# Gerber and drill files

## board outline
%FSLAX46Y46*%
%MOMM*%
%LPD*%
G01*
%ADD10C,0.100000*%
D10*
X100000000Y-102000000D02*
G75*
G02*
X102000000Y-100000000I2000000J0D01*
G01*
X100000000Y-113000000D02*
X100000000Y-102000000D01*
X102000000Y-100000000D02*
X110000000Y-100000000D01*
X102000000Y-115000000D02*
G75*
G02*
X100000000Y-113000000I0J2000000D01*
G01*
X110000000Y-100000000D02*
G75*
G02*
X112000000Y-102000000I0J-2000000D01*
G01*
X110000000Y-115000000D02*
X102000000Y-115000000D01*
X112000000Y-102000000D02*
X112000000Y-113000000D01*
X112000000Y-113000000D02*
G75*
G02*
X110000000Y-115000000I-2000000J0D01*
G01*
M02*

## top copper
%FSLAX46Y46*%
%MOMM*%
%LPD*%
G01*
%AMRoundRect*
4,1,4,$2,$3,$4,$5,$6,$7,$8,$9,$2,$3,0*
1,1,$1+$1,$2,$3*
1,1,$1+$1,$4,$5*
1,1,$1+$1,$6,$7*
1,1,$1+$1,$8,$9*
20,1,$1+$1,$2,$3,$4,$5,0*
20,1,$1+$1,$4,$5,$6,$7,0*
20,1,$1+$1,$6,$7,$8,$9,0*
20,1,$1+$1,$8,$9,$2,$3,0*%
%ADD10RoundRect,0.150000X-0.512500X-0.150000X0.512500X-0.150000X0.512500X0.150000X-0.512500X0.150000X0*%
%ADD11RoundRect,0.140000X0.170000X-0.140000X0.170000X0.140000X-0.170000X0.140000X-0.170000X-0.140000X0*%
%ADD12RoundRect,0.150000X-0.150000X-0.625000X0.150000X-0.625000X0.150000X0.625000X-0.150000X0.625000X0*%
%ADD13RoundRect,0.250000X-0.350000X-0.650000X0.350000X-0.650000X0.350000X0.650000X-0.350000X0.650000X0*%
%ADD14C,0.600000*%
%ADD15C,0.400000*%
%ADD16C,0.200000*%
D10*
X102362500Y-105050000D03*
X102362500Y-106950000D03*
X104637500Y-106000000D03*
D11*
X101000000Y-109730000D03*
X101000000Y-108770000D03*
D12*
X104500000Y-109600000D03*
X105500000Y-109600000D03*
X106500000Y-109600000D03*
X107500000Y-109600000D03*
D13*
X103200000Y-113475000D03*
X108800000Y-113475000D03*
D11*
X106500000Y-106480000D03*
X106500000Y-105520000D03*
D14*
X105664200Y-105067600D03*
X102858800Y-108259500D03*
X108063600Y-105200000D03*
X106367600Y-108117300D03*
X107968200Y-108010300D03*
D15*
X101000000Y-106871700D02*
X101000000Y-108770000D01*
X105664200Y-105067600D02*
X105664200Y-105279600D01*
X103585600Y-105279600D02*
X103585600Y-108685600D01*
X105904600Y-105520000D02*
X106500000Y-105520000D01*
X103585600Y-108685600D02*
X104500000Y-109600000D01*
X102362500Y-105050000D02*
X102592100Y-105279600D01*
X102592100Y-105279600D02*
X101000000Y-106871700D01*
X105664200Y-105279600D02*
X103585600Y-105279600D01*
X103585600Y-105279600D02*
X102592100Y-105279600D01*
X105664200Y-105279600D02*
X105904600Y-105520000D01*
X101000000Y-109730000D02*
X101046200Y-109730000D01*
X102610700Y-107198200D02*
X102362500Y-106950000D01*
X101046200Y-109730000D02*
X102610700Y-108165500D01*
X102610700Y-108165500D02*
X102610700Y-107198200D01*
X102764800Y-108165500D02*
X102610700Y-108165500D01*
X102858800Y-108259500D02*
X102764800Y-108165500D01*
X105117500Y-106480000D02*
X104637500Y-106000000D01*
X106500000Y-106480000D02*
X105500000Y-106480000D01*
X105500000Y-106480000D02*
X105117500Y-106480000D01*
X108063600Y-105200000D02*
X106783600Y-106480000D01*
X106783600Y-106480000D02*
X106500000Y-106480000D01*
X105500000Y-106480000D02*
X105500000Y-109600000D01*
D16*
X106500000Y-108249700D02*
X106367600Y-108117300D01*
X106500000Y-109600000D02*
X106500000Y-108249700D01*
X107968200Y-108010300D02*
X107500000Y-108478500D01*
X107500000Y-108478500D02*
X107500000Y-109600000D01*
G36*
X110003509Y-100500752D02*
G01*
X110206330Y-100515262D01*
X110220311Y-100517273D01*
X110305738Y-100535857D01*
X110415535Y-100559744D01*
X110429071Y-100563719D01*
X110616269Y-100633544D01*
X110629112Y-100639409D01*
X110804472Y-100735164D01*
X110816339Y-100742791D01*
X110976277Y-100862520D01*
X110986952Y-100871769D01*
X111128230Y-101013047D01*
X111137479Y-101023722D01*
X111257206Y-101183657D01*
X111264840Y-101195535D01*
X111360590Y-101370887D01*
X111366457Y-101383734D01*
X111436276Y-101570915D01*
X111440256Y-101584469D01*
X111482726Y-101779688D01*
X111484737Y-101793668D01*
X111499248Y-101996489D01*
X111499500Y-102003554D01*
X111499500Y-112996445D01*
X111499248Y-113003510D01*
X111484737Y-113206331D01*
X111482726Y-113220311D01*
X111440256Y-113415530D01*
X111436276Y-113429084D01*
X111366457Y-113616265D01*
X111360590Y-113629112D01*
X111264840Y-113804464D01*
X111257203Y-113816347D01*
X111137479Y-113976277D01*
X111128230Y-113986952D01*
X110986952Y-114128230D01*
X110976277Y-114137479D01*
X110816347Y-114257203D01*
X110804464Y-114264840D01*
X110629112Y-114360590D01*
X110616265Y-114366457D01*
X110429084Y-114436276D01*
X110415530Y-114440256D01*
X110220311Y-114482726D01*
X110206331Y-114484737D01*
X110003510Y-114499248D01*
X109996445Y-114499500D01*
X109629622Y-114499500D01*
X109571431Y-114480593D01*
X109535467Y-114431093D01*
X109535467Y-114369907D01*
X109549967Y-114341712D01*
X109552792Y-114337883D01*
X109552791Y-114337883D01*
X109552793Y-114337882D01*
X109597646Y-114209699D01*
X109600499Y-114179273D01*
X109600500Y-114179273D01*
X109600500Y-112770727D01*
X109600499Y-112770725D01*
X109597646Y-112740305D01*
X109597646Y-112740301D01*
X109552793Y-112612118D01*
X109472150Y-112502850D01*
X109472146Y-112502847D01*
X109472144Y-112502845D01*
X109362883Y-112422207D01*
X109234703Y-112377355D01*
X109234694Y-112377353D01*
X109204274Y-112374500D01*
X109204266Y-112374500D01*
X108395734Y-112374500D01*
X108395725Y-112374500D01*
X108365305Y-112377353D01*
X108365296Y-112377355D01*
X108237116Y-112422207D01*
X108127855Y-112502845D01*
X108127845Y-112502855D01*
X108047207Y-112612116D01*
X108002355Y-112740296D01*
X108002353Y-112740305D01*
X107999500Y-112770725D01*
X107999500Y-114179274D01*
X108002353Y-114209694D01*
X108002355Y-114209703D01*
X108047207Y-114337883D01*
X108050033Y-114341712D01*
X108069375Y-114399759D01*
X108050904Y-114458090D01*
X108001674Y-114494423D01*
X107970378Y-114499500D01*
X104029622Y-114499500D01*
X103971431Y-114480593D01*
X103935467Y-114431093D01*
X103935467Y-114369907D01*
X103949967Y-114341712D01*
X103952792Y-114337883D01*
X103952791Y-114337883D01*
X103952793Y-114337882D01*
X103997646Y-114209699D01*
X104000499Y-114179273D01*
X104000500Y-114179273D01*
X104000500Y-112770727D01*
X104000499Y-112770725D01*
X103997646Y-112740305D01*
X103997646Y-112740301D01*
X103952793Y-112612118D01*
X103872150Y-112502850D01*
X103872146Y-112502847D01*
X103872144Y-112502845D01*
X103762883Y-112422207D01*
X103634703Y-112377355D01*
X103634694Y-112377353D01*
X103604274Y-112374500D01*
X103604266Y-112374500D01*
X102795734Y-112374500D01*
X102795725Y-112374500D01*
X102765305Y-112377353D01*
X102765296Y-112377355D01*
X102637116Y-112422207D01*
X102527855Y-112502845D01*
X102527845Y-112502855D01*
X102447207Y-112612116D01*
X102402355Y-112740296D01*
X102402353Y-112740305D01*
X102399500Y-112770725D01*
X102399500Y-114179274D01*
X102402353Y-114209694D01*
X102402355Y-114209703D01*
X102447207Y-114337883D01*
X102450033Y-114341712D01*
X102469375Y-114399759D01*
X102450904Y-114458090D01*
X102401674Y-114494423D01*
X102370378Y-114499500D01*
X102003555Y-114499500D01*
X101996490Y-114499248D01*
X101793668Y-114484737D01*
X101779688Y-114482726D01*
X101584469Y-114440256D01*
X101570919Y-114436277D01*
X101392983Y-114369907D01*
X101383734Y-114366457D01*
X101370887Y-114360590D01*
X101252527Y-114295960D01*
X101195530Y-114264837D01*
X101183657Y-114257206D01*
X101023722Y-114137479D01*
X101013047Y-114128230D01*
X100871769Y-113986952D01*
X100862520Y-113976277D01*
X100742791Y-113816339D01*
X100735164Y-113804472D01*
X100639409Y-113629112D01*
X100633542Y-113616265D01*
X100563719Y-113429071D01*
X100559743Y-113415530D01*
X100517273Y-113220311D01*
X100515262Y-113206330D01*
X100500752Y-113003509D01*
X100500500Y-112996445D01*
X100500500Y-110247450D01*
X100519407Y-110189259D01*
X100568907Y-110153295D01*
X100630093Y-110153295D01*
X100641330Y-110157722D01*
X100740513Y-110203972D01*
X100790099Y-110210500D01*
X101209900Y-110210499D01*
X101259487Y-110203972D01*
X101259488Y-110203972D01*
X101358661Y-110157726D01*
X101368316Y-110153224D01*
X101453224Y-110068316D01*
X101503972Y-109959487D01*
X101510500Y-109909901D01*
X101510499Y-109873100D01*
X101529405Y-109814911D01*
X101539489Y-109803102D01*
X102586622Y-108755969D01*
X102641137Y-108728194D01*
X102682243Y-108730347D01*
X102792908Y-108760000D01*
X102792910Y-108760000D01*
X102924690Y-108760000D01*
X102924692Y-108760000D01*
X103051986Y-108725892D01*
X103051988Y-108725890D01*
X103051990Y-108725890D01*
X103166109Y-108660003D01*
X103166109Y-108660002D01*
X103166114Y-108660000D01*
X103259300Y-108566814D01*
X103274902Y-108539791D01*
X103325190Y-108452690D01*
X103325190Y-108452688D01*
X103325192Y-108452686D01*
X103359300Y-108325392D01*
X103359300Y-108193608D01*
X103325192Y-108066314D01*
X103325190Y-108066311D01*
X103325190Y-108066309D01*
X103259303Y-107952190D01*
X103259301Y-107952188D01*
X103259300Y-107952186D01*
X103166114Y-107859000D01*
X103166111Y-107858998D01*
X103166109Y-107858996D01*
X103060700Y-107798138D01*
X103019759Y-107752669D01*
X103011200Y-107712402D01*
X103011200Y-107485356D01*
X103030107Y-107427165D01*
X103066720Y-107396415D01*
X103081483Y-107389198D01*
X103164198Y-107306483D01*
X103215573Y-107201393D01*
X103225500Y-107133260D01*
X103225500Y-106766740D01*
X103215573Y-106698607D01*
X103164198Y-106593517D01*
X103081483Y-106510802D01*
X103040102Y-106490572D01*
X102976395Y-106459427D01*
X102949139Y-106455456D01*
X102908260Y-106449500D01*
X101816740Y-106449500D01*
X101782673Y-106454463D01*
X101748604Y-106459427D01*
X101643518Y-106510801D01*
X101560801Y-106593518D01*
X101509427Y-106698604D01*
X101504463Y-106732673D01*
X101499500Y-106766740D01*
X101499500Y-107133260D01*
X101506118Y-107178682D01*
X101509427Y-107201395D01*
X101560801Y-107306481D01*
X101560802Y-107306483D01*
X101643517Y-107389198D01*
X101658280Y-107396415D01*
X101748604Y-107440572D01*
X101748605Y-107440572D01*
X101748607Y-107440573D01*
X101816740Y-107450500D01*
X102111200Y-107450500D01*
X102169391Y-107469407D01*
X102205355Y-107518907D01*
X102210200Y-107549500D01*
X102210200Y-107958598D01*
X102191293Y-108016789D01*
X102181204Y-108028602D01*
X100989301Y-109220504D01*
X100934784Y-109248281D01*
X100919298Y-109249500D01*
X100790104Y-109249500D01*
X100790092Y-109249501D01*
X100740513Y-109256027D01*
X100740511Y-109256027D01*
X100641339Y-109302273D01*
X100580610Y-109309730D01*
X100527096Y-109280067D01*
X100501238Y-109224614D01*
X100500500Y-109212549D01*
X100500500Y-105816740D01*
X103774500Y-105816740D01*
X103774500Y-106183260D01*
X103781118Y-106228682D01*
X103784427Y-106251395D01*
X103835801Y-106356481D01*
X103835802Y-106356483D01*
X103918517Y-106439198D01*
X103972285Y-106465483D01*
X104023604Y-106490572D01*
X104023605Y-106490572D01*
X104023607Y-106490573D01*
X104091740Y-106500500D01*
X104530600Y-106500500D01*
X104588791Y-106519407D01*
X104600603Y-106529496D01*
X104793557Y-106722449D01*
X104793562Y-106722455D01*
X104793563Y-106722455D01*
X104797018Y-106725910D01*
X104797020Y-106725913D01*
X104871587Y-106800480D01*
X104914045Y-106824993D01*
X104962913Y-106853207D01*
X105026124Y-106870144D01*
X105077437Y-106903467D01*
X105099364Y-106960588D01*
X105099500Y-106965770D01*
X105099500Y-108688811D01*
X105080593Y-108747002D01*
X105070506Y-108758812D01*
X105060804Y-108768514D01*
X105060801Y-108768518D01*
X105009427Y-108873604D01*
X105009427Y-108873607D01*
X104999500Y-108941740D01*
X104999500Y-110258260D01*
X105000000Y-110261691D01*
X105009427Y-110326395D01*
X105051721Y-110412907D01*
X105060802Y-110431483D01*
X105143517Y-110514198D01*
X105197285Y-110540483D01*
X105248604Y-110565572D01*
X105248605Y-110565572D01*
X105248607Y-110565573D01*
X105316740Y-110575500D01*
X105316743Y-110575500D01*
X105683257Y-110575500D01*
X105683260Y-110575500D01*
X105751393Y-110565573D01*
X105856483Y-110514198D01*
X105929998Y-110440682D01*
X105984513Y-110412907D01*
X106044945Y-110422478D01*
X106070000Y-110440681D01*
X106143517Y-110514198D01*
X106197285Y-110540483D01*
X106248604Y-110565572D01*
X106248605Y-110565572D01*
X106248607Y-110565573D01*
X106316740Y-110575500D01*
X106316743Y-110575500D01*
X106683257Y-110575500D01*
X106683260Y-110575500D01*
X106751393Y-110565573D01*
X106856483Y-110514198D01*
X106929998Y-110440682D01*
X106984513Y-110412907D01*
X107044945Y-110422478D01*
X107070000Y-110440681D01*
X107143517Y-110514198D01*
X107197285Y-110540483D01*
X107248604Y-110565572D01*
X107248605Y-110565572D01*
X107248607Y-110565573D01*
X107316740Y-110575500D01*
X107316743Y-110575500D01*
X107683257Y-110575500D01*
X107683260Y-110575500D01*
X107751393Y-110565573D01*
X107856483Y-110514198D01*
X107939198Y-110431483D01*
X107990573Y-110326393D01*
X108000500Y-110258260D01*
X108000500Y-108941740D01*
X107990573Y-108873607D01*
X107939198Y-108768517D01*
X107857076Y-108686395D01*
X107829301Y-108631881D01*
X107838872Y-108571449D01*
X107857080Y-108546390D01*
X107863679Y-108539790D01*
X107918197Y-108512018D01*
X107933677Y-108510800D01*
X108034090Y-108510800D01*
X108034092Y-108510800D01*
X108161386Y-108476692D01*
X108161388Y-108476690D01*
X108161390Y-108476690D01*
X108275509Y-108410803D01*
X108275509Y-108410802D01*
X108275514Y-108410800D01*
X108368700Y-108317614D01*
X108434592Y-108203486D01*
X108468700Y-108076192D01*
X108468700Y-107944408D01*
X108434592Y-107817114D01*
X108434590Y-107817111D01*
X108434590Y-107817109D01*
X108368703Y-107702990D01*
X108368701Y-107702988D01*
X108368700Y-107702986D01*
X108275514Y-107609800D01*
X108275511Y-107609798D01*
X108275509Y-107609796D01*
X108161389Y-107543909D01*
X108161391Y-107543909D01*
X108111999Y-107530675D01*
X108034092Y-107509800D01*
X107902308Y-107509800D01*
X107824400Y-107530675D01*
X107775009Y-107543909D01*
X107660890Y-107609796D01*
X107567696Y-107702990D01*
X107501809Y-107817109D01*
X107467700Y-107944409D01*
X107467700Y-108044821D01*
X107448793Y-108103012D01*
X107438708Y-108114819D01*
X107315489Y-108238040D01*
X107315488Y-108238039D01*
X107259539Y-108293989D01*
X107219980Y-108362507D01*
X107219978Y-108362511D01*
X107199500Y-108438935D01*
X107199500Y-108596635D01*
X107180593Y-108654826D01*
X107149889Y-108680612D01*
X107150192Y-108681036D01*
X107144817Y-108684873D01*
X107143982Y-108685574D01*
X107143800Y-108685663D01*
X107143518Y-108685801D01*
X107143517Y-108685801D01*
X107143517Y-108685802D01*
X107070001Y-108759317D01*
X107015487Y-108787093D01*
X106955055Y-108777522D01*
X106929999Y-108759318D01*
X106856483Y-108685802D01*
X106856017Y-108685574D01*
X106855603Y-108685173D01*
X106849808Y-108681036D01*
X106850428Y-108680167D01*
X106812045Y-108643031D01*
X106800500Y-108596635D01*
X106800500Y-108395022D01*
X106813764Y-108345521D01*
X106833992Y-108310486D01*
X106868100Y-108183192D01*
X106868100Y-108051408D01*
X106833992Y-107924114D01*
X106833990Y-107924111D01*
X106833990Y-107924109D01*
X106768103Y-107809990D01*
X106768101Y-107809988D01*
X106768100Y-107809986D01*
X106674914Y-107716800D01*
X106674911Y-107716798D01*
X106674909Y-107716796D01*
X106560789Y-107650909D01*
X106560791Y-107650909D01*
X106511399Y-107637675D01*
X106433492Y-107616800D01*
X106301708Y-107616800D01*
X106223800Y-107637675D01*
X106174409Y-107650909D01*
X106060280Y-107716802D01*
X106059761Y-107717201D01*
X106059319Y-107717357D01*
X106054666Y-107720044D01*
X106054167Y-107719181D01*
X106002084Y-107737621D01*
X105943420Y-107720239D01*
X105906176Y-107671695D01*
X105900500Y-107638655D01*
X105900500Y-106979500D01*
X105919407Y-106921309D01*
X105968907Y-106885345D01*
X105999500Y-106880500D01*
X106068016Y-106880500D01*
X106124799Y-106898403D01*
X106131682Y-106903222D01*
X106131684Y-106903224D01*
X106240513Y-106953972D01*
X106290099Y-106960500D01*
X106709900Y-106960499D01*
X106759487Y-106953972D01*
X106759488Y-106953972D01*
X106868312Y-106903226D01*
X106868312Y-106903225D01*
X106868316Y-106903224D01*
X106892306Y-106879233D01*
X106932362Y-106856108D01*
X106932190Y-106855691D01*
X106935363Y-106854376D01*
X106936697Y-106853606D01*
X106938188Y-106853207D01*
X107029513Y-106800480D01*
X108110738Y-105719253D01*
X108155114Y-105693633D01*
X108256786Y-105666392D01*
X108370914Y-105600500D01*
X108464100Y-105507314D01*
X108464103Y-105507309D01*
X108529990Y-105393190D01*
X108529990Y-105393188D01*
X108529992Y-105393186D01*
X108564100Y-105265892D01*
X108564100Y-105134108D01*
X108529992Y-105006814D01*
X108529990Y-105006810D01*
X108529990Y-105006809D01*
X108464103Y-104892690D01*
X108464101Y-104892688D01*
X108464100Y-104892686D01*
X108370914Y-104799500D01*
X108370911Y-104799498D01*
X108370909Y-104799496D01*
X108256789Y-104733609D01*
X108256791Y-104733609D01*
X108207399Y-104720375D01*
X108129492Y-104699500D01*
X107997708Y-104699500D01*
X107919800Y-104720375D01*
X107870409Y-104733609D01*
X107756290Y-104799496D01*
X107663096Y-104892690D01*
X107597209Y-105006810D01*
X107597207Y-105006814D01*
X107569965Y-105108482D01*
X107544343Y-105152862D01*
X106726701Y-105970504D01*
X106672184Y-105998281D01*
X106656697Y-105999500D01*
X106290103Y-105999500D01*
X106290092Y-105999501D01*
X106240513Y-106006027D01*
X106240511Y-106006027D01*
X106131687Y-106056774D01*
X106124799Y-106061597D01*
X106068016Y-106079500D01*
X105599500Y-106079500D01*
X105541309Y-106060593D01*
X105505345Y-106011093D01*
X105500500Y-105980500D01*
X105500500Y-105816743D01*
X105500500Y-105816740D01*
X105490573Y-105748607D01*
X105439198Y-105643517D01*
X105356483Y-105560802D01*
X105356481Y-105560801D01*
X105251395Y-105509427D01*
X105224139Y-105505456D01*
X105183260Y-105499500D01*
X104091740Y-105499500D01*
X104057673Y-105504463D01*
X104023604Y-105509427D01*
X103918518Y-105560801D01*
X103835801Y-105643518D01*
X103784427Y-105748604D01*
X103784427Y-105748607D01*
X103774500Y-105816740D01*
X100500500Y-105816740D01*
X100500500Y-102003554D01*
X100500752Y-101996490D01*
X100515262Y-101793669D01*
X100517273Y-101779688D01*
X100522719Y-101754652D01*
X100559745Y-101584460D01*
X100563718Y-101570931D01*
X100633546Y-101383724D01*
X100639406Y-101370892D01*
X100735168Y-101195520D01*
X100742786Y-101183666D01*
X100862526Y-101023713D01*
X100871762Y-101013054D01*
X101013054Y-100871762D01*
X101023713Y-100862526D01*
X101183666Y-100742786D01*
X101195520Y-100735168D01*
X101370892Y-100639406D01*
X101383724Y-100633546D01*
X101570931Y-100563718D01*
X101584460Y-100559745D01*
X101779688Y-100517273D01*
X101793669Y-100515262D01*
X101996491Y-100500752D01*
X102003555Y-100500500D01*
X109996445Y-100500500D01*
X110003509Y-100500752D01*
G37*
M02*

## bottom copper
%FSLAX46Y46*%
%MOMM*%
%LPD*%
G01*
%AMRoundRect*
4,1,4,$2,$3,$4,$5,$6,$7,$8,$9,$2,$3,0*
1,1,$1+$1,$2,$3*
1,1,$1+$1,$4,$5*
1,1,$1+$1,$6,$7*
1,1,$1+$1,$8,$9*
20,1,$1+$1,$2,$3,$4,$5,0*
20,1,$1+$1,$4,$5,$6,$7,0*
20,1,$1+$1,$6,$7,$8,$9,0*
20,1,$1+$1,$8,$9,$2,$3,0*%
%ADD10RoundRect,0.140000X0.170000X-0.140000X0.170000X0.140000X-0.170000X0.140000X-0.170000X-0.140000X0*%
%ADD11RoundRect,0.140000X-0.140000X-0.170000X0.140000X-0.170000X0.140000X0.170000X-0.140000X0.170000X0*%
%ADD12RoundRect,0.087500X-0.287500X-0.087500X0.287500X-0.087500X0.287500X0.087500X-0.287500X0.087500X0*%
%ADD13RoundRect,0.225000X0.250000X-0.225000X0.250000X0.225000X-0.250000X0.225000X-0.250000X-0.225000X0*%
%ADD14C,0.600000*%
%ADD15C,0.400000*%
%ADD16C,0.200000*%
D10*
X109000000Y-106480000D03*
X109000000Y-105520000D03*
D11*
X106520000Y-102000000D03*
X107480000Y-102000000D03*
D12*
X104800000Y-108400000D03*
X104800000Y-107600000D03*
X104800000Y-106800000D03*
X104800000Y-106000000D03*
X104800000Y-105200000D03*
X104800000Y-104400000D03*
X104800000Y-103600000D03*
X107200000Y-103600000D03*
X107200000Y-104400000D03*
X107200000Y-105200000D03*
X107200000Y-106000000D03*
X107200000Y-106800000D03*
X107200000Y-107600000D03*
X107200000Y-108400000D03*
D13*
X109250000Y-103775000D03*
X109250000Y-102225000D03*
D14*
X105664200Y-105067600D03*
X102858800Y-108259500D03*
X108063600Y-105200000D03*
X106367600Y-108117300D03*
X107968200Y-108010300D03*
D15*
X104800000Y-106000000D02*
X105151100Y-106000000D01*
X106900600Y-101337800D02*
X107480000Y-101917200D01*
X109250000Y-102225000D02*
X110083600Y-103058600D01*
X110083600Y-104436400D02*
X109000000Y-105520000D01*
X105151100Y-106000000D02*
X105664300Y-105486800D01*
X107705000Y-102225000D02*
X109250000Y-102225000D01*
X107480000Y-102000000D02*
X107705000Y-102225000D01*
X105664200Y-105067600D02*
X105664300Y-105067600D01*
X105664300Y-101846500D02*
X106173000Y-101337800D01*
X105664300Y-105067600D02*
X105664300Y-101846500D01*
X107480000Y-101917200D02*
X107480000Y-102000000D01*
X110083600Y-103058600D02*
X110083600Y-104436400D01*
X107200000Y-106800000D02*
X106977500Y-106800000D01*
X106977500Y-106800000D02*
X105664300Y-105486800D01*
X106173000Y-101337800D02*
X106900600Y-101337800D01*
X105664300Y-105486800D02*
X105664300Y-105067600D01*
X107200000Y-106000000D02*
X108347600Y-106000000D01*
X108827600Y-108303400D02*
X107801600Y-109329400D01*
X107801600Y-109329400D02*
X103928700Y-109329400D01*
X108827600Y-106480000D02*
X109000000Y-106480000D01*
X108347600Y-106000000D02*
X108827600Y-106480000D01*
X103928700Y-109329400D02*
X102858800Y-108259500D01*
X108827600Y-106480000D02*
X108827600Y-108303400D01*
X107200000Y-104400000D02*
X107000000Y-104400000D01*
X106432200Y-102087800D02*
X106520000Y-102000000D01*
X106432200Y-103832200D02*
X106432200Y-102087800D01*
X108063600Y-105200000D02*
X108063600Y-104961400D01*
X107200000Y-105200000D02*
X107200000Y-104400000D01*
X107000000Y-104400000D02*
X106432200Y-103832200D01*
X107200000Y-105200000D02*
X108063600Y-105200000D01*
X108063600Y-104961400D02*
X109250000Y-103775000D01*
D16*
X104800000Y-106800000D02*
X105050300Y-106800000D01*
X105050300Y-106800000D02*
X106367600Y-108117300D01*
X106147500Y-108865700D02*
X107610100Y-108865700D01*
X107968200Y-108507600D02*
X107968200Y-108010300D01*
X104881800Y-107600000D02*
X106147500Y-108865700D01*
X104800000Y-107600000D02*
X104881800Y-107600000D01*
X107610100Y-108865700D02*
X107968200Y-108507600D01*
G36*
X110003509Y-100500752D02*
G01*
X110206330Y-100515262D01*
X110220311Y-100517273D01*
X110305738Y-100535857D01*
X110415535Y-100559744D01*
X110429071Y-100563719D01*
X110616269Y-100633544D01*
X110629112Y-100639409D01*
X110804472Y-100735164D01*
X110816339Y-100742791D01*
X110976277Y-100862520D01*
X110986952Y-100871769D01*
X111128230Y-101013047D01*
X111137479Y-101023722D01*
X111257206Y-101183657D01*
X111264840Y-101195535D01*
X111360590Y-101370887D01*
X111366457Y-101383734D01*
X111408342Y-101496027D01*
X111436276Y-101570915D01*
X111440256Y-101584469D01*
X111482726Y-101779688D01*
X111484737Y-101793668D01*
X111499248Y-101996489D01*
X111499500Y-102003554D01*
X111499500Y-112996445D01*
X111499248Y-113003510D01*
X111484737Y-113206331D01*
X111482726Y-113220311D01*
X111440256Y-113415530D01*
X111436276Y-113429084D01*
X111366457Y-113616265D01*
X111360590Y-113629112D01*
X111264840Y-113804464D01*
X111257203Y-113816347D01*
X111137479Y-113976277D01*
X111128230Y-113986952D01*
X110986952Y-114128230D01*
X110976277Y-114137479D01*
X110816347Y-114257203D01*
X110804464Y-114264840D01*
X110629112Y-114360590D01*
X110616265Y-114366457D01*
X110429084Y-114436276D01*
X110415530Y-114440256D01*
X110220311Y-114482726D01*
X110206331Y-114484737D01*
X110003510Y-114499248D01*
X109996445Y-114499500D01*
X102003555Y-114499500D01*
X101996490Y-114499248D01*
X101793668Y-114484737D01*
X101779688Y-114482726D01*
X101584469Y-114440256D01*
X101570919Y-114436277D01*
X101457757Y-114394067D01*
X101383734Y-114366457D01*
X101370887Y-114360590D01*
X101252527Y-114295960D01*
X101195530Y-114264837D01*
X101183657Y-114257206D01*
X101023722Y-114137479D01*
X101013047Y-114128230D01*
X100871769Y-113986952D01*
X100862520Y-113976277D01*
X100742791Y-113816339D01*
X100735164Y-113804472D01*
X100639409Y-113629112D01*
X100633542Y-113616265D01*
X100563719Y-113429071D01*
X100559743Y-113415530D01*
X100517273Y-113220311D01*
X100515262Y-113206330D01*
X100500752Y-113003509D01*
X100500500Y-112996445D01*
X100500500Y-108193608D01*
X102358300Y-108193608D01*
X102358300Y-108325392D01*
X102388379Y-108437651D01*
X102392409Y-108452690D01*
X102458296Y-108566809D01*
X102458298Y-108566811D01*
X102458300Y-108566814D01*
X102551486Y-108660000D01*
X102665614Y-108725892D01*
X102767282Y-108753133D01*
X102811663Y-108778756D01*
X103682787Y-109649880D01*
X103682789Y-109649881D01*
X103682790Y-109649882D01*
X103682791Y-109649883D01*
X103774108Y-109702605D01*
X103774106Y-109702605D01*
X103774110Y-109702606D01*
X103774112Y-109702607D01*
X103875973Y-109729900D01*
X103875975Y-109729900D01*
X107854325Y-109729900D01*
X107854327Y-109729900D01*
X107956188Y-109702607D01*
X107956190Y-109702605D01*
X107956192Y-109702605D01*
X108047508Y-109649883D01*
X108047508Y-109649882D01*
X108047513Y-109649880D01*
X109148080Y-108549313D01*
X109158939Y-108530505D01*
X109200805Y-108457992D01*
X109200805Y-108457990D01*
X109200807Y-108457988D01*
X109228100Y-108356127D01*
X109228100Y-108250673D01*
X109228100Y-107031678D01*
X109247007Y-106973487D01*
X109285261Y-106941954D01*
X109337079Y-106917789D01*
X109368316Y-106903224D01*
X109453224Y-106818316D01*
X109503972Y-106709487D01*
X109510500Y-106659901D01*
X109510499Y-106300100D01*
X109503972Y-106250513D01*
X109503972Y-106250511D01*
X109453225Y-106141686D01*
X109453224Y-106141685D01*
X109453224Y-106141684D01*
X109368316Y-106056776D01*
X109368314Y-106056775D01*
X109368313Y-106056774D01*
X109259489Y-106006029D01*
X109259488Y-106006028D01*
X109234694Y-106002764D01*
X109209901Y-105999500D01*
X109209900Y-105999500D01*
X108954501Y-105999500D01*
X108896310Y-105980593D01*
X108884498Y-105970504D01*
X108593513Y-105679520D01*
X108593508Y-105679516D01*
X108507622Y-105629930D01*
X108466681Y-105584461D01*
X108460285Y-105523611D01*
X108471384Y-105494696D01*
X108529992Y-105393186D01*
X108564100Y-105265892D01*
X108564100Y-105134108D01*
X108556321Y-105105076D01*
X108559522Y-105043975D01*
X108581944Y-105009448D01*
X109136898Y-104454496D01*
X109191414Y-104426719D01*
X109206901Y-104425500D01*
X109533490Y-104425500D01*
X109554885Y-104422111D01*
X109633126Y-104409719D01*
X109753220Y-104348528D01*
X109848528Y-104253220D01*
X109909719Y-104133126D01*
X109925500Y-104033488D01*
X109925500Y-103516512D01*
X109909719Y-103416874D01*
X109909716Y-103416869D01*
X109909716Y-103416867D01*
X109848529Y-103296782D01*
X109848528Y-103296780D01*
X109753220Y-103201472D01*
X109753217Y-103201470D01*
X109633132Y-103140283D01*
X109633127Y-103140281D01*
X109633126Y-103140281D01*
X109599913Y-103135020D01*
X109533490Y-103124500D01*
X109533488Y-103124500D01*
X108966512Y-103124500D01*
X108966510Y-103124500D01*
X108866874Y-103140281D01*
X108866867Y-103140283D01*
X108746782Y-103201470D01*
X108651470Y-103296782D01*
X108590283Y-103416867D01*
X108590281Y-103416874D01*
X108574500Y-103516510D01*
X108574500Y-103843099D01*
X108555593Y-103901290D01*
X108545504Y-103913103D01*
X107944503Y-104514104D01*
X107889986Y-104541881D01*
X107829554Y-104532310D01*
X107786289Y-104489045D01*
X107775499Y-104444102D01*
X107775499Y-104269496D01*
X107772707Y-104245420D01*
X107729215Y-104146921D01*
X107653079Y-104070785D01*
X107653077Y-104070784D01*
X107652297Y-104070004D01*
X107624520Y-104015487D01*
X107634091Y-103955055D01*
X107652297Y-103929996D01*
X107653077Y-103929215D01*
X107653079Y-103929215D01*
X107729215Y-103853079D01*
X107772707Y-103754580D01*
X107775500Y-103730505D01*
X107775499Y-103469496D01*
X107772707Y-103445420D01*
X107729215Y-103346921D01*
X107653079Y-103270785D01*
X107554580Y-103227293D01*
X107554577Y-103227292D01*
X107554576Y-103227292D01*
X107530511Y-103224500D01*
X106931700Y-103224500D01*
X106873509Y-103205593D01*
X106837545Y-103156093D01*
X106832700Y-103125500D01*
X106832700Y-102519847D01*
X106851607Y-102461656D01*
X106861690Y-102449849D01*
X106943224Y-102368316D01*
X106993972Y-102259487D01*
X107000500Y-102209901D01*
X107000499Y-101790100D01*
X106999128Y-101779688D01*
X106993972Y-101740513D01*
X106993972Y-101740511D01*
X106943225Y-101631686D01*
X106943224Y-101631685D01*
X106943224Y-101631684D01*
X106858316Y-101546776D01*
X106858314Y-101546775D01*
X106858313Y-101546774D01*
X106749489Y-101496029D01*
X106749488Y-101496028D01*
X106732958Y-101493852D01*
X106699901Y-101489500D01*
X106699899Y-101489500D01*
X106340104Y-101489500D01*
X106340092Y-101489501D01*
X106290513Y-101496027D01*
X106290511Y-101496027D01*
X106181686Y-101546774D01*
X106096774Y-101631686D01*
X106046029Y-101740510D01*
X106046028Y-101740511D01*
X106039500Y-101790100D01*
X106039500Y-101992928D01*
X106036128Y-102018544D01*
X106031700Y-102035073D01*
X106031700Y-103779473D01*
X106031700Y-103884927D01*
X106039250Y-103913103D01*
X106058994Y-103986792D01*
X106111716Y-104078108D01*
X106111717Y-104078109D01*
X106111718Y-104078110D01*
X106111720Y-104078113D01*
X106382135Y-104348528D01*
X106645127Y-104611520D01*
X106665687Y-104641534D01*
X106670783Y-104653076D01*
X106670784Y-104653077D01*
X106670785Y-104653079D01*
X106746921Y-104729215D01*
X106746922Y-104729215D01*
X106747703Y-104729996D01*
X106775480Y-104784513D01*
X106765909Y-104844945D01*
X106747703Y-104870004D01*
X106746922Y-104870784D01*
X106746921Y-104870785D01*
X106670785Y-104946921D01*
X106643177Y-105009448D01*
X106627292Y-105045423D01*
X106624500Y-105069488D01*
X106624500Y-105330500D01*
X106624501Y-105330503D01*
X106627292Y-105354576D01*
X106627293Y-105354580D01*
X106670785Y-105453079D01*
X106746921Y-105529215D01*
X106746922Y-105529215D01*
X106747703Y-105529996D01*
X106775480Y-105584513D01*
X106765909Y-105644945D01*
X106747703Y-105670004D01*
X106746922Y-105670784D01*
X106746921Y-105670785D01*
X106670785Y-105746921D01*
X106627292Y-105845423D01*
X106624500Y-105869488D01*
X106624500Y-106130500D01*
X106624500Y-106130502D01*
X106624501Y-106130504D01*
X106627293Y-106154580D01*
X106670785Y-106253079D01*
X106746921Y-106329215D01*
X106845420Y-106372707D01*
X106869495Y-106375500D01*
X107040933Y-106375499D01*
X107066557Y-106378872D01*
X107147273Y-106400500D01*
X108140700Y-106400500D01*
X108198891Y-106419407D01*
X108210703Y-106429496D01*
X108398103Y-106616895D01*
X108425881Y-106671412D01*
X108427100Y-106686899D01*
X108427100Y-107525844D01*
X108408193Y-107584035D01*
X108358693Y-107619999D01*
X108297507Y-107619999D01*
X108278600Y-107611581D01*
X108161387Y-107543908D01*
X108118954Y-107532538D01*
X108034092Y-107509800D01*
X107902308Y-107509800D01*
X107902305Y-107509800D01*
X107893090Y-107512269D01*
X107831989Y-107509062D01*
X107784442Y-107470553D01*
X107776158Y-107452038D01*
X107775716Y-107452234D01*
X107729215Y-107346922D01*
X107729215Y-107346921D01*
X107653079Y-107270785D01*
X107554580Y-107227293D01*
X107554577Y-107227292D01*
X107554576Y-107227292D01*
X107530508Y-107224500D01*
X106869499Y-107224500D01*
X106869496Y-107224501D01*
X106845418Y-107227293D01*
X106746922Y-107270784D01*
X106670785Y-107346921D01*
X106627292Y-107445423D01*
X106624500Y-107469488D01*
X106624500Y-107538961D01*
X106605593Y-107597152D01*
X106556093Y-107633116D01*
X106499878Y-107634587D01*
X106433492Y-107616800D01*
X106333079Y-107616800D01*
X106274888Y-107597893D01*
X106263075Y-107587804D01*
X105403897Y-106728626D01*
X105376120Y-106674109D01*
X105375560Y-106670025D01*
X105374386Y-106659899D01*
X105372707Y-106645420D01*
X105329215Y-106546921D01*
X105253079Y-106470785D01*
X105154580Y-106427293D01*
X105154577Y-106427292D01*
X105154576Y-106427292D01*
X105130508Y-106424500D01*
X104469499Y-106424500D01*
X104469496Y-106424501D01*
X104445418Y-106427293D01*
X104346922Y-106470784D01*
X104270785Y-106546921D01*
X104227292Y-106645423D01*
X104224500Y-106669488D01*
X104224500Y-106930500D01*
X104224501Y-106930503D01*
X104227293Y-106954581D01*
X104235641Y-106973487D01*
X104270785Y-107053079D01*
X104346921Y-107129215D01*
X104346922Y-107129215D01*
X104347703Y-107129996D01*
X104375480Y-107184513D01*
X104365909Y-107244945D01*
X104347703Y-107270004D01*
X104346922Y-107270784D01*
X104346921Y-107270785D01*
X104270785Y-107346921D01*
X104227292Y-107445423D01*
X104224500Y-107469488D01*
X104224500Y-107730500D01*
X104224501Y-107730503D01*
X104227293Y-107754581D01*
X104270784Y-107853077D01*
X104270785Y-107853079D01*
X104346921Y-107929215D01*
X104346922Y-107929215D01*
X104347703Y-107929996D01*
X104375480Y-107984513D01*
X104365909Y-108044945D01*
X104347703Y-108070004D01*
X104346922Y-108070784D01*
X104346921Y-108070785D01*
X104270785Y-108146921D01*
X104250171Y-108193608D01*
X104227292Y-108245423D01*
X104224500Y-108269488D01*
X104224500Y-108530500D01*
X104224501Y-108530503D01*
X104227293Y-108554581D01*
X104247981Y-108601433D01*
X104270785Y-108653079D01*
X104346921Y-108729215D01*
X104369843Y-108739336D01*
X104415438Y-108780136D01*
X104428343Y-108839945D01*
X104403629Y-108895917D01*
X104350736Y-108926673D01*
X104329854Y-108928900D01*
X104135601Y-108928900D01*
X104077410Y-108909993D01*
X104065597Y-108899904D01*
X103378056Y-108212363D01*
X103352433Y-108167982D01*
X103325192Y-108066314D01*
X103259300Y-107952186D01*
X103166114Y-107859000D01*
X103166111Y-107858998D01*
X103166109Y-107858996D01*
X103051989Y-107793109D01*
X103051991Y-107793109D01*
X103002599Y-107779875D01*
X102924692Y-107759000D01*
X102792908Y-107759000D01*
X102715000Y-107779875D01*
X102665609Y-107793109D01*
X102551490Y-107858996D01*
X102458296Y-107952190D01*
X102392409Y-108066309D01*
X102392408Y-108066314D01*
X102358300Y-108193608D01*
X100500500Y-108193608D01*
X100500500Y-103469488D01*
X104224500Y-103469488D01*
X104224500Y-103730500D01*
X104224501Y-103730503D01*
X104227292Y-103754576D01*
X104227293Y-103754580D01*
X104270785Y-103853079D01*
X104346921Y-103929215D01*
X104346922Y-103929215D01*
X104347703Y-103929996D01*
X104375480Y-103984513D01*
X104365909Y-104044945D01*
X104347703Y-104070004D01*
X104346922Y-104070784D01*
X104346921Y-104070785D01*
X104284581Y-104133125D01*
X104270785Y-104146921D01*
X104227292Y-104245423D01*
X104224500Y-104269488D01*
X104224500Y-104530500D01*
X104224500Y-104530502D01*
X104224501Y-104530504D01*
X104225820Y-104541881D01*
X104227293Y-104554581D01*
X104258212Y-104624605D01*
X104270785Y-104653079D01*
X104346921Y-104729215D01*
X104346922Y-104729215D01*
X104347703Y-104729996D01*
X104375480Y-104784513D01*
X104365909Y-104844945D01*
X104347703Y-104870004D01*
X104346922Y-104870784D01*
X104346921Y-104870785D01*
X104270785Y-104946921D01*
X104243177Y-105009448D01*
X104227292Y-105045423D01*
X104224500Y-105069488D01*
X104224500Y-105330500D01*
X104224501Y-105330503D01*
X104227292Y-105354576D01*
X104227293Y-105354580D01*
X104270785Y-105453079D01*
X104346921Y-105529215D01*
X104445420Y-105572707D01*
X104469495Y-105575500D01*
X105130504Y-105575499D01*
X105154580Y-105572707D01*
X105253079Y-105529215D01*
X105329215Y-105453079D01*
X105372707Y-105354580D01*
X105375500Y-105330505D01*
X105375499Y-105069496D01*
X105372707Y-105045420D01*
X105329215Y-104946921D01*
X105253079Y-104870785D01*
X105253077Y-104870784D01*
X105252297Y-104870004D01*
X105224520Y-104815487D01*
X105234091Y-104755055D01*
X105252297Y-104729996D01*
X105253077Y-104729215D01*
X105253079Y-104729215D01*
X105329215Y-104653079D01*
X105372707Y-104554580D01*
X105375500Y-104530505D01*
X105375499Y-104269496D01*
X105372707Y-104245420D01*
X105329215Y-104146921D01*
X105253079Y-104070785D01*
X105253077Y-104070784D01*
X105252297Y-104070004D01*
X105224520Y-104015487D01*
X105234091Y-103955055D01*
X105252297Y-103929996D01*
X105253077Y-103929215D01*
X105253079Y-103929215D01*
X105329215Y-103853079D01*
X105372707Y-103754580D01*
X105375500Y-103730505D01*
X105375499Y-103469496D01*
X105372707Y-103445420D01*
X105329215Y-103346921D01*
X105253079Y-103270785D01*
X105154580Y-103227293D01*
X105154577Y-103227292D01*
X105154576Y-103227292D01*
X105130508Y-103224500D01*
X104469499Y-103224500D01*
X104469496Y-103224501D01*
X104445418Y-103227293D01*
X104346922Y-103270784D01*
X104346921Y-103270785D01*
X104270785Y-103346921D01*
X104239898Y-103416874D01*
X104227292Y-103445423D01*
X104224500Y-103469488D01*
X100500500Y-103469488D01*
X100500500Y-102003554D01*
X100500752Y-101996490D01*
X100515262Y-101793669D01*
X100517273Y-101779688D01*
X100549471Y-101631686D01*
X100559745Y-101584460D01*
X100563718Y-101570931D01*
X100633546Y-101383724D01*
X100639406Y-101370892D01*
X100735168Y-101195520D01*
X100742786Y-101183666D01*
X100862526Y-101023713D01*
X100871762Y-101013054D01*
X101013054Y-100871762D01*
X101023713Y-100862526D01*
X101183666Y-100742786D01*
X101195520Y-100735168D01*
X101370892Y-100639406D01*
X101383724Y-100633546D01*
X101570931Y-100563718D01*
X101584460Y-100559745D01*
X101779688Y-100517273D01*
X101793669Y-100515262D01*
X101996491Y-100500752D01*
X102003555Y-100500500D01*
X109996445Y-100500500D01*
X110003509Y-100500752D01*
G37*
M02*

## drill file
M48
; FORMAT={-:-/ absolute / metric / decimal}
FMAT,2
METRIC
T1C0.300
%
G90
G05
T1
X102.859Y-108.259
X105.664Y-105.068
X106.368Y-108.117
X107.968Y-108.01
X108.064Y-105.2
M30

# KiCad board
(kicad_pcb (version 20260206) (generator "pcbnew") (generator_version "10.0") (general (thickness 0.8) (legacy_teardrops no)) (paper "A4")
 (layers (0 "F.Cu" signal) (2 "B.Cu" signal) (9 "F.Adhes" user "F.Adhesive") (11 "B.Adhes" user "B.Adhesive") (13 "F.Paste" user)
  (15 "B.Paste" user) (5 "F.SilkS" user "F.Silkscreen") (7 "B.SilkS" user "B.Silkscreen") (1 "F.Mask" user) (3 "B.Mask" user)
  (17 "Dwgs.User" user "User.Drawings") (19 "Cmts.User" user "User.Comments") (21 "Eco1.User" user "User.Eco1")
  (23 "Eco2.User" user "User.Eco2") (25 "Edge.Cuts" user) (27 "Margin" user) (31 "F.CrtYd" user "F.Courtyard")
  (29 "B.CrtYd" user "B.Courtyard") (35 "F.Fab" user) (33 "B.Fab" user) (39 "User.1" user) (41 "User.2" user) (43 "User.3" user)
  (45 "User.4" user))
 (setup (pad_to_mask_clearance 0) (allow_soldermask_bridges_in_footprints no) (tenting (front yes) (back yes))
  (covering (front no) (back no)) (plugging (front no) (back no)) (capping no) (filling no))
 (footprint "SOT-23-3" (layer "F.Cu") (at 103.5 106)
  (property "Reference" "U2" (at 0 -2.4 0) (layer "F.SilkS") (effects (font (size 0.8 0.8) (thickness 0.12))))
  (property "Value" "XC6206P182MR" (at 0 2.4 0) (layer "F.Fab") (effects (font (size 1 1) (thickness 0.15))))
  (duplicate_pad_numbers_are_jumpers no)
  (pad "1" smd roundrect (at -1.1375 -0.95) (size 1.325 0.6) (layers "F.Cu" "F.Mask" "F.Paste") (roundrect_rratio 0.25) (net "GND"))
  (pad "2" smd roundrect (at -1.1375 0.95) (size 1.325 0.6) (layers "F.Cu" "F.Mask" "F.Paste") (roundrect_rratio 0.25) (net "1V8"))
  (pad "3" smd roundrect (at 1.1375 0) (size 1.325 0.6) (layers "F.Cu" "F.Mask" "F.Paste") (roundrect_rratio 0.25) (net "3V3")))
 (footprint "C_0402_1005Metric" (layer "F.Cu") (at 101 109.25 90)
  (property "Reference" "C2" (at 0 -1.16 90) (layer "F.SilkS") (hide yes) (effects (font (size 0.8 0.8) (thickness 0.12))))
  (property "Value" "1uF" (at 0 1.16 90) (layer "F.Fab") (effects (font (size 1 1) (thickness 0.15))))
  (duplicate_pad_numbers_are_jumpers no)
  (pad "1" smd roundrect (at -0.48 0 90) (size 0.56 0.62) (layers "F.Cu" "F.Mask" "F.Paste") (roundrect_rratio 0.25) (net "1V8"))
  (pad "2" smd roundrect (at 0.48 0 90) (size 0.56 0.62) (layers "F.Cu" "F.Mask" "F.Paste") (roundrect_rratio 0.25) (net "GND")))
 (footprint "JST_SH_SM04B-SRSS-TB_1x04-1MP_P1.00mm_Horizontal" (layer "F.Cu") (at 106 111.6)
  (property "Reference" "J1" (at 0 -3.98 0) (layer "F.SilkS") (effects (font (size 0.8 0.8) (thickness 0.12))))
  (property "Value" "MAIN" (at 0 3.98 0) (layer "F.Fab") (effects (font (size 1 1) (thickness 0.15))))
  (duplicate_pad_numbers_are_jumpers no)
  (pad "1" smd roundrect (at -1.5 -2) (size 0.6 1.55) (layers "F.Cu" "F.Mask" "F.Paste") (roundrect_rratio 0.25) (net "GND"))
  (pad "2" smd roundrect (at -0.5 -2) (size 0.6 1.55) (layers "F.Cu" "F.Mask" "F.Paste") (roundrect_rratio 0.25) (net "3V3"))
  (pad "3" smd roundrect (at 0.5 -2) (size 0.6 1.55) (layers "F.Cu" "F.Mask" "F.Paste") (roundrect_rratio 0.25) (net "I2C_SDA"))
  (pad "4" smd roundrect (at 1.5 -2) (size 0.6 1.55) (layers "F.Cu" "F.Mask" "F.Paste") (roundrect_rratio 0.25) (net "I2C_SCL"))
  (pad "MP" smd roundrect (at -2.8 1.875) (size 1.2 1.8) (layers "F.Cu" "F.Mask" "F.Paste") (roundrect_rratio 0.208333))
  (pad "MP" smd roundrect (at 2.8 1.875) (size 1.2 1.8) (layers "F.Cu" "F.Mask" "F.Paste") (roundrect_rratio 0.208333)))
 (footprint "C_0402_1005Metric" (layer "F.Cu") (at 106.5 106 90)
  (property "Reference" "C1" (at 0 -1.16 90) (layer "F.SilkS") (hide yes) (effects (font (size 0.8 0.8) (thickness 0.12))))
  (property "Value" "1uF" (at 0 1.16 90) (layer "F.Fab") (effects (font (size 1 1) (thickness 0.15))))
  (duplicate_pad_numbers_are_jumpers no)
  (pad "1" smd roundrect (at -0.48 0 90) (size 0.56 0.62) (layers "F.Cu" "F.Mask" "F.Paste") (roundrect_rratio 0.25) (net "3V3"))
  (pad "2" smd roundrect (at 0.48 0 90) (size 0.56 0.62) (layers "F.Cu" "F.Mask" "F.Paste") (roundrect_rratio 0.25) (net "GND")))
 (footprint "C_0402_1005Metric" (layer "B.Cu") (at 109 106 90)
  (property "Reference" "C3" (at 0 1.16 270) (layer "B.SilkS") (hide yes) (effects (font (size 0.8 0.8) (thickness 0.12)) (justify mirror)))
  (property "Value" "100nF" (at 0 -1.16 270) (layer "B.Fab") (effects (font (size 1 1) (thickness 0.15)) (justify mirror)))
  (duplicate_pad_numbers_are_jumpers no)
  (pad "1" smd roundrect (at -0.48 0 90) (size 0.56 0.62) (layers "B.Cu" "B.Mask" "B.Paste") (roundrect_rratio 0.25) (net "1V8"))
  (pad "2" smd roundrect (at 0.48 0 90) (size 0.56 0.62) (layers "B.Cu" "B.Mask" "B.Paste") (roundrect_rratio 0.25) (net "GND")))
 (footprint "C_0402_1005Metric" (layer "B.Cu") (at 107 102)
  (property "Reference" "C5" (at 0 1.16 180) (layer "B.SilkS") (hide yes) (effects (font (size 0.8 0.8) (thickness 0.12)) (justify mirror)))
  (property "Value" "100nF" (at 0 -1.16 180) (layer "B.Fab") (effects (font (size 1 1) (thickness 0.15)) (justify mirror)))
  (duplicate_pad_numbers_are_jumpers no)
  (pad "1" smd roundrect (at -0.48 0) (size 0.56 0.62) (layers "B.Cu" "B.Mask" "B.Paste") (roundrect_rratio 0.25) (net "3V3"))
  (pad "2" smd roundrect (at 0.48 0) (size 0.56 0.62) (layers "B.Cu" "B.Mask" "B.Paste") (roundrect_rratio 0.25) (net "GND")))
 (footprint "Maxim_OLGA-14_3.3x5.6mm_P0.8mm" (layer "B.Cu") (at 106 106)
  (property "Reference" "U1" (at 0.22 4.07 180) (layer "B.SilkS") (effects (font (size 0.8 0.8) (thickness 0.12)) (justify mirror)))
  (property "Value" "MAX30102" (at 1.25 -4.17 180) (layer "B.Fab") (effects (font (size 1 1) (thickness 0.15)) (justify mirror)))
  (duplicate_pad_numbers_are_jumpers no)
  (pad "1" smd roundrect (at -1.2 2.4) (size 0.75 0.35) (layers "B.Cu" "B.Mask" "B.Paste") (roundrect_rratio 0.25))
  (pad "2" smd roundrect (at -1.2 1.6) (size 0.75 0.35) (layers "B.Cu" "B.Mask" "B.Paste") (roundrect_rratio 0.25) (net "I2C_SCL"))
  (pad "3" smd roundrect (at -1.2 0.8) (size 0.75 0.35) (layers "B.Cu" "B.Mask" "B.Paste") (roundrect_rratio 0.25) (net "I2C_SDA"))
  (pad "4" smd roundrect (at -1.2 0) (size 0.75 0.35) (layers "B.Cu" "B.Mask" "B.Paste") (roundrect_rratio 0.25) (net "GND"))
  (pad "5" smd roundrect (at -1.2 -0.8) (size 0.75 0.35) (layers "B.Cu" "B.Mask" "B.Paste") (roundrect_rratio 0.25))
  (pad "6" smd roundrect (at -1.2 -1.6) (size 0.75 0.35) (layers "B.Cu" "B.Mask" "B.Paste") (roundrect_rratio 0.25))
  (pad "7" smd roundrect (at -1.2 -2.4) (size 0.75 0.35) (layers "B.Cu" "B.Mask" "B.Paste") (roundrect_rratio 0.25))
  (pad "8" smd roundrect (at 1.2 -2.4) (size 0.75 0.35) (layers "B.Cu" "B.Mask" "B.Paste") (roundrect_rratio 0.25))
  (pad "9" smd roundrect (at 1.2 -1.6) (size 0.75 0.35) (layers "B.Cu" "B.Mask" "B.Paste") (roundrect_rratio 0.25) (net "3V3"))
  (pad "10" smd roundrect (at 1.2 -0.8) (size 0.75 0.35) (layers "B.Cu" "B.Mask" "B.Paste") (roundrect_rratio 0.25) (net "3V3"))
  (pad "11" smd roundrect (at 1.2 0) (size 0.75 0.35) (layers "B.Cu" "B.Mask" "B.Paste") (roundrect_rratio 0.25) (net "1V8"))
  (pad "12" smd roundrect (at 1.2 0.8) (size 0.75 0.35) (layers "B.Cu" "B.Mask" "B.Paste") (roundrect_rratio 0.25) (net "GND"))
  (pad "13" smd roundrect (at 1.2 1.6) (size 0.75 0.35) (layers "B.Cu" "B.Mask" "B.Paste") (roundrect_rratio 0.25))
  (pad "14" smd roundrect (at 1.2 2.4) (size 0.75 0.35) (layers "B.Cu" "B.Mask" "B.Paste") (roundrect_rratio 0.25)))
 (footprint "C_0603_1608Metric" (layer "B.Cu") (at 109.25 103 90)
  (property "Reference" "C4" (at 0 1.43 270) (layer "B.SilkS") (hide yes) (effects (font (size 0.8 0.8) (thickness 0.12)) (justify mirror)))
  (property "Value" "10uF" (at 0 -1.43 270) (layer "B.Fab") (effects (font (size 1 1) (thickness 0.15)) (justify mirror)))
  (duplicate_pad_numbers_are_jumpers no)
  (pad "1" smd roundrect (at -0.775 0 90) (size 0.9 0.95) (layers "B.Cu" "B.Mask" "B.Paste") (roundrect_rratio 0.25) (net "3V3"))
  (pad "2" smd roundrect (at 0.775 0 90) (size 0.9 0.95) (layers "B.Cu" "B.Mask" "B.Paste") (roundrect_rratio 0.25) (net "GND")))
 (gr_arc (start 100 102) (mid 100.5858 100.5858) (end 102 100) (stroke (width 0.1) (type default)) (layer "Edge.Cuts"))
 (gr_line (start 100 113) (end 100 102) (stroke (width 0.1) (type default)) (layer "Edge.Cuts"))
 (gr_line (start 102 100) (end 110 100) (stroke (width 0.1) (type default)) (layer "Edge.Cuts"))
 (gr_arc (start 102 115) (mid 100.5858 114.4142) (end 100 113) (stroke (width 0.1) (type default)) (layer "Edge.Cuts"))
 (gr_arc (start 110 100) (mid 111.4142 100.5858) (end 112 102) (stroke (width 0.1) (type default)) (layer "Edge.Cuts"))
 (gr_line (start 110 115) (end 102 115) (stroke (width 0.1) (type default)) (layer "Edge.Cuts"))
 (gr_line (start 112 102) (end 112 113) (stroke (width 0.1) (type default)) (layer "Edge.Cuts"))
 (gr_arc (start 112 113) (mid 111.4142 114.4142) (end 110 115) (stroke (width 0.1) (type default)) (layer "Edge.Cuts"))
 (segment (start 101 106.8717) (end 101 108.77) (width 0.4) (layer "F.Cu") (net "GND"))
 (segment (start 105.6642 105.0676) (end 105.6642 105.2796) (width 0.4) (layer "F.Cu") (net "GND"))
 (segment (start 103.5856 105.2796) (end 103.5856 108.6856) (width 0.4) (layer "F.Cu") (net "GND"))
 (segment (start 105.9046 105.52) (end 106.5 105.52) (width 0.4) (layer "F.Cu") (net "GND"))
 (segment (start 103.5856 108.6856) (end 104.5 109.6) (width 0.4) (layer "F.Cu") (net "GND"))
 (segment (start 102.3625 105.05) (end 102.5921 105.2796) (width 0.4) (layer "F.Cu") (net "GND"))
 (segment (start 102.5921 105.2796) (end 101 106.8717) (width 0.4) (layer "F.Cu") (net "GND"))
 (segment (start 105.6642 105.2796) (end 103.5856 105.2796) (width 0.4) (layer "F.Cu") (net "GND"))
 (segment (start 103.5856 105.2796) (end 102.5921 105.2796) (width 0.4) (layer "F.Cu") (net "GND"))
 (segment (start 105.6642 105.2796) (end 105.9046 105.52) (width 0.4) (layer "F.Cu") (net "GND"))
 (via (at 105.6642 105.0676) (size 0.6) (drill 0.3) (layers "F.Cu" "B.Cu") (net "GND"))
 (segment (start 104.8 106) (end 105.1511 106) (width 0.4) (layer "B.Cu") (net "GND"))
 (segment (start 106.9006 101.3378) (end 107.48 101.9172) (width 0.4) (layer "B.Cu") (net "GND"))
 (segment (start 109.25 102.225) (end 110.0836 103.0586) (width 0.4) (layer "B.Cu") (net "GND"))
 (segment (start 110.0836 104.4364) (end 109 105.52) (width 0.4) (layer "B.Cu") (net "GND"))
 (segment (start 105.1511 106) (end 105.6643 105.4868) (width 0.4) (layer "B.Cu") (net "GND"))
 (segment (start 107.705 102.225) (end 109.25 102.225) (width 0.4) (layer "B.Cu") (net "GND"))
 (segment (start 107.48 102) (end 107.705 102.225) (width 0.4) (layer "B.Cu") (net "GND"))
 (segment (start 105.6642 105.0676) (end 105.6643 105.0676) (width 0.4) (layer "B.Cu") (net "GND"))
 (segment (start 105.6643 101.8465) (end 106.173 101.3378) (width 0.4) (layer "B.Cu") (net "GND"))
 (segment (start 105.6643 105.0676) (end 105.6643 101.8465) (width 0.4) (layer "B.Cu") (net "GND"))
 (segment (start 107.48 101.9172) (end 107.48 102) (width 0.4) (layer "B.Cu") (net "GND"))
 (segment (start 110.0836 103.0586) (end 110.0836 104.4364) (width 0.4) (layer "B.Cu") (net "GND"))
 (segment (start 107.2 106.8) (end 106.9775 106.8) (width 0.4) (layer "B.Cu") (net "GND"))
 (segment (start 106.9775 106.8) (end 105.6643 105.4868) (width 0.4) (layer "B.Cu") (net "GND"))
 (segment (start 106.173 101.3378) (end 106.9006 101.3378) (width 0.4) (layer "B.Cu") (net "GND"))
 (segment (start 105.6643 105.4868) (end 105.6643 105.0676) (width 0.4) (layer "B.Cu") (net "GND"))
 (segment (start 101 109.73) (end 101.0462 109.73) (width 0.4) (layer "F.Cu") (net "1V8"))
 (segment (start 102.6107 107.1982) (end 102.3625 106.95) (width 0.4) (layer "F.Cu") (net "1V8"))
 (segment (start 101.0462 109.73) (end 102.6107 108.1655) (width 0.4) (layer "F.Cu") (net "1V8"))
 (segment (start 102.6107 108.1655) (end 102.6107 107.1982) (width 0.4) (layer "F.Cu") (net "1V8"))
 (segment (start 102.7648 108.1655) (end 102.6107 108.1655) (width 0.4) (layer "F.Cu") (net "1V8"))
 (segment (start 102.8588 108.2595) (end 102.7648 108.1655) (width 0.4) (layer "F.Cu") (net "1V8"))
 (via (at 102.8588 108.2595) (size 0.6) (drill 0.3) (layers "F.Cu" "B.Cu") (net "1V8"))
 (segment (start 107.2 106) (end 108.3476 106) (width 0.4) (layer "B.Cu") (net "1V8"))
 (segment (start 108.8276 108.3034) (end 107.8016 109.3294) (width 0.4) (layer "B.Cu") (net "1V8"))
 (segment (start 107.8016 109.3294) (end 103.9287 109.3294) (width 0.4) (layer "B.Cu") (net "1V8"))
 (segment (start 108.8276 106.48) (end 109 106.48) (width 0.4) (layer "B.Cu") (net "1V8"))
 (segment (start 108.3476 106) (end 108.8276 106.48) (width 0.4) (layer "B.Cu") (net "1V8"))
 (segment (start 103.9287 109.3294) (end 102.8588 108.2595) (width 0.4) (layer "B.Cu") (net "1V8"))
 (segment (start 108.8276 106.48) (end 108.8276 108.3034) (width 0.4) (layer "B.Cu") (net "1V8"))
 (segment (start 105.1175 106.48) (end 104.6375 106) (width 0.4) (layer "F.Cu") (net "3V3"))
 (segment (start 106.5 106.48) (end 105.5 106.48) (width 0.4) (layer "F.Cu") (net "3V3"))
 (segment (start 105.5 106.48) (end 105.1175 106.48) (width 0.4) (layer "F.Cu") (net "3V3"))
 (segment (start 108.0636 105.2) (end 106.7836 106.48) (width 0.4) (layer "F.Cu") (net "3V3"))
 (segment (start 106.7836 106.48) (end 106.5 106.48) (width 0.4) (layer "F.Cu") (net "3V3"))
 (segment (start 105.5 106.48) (end 105.5 109.6) (width 0.4) (layer "F.Cu") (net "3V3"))
 (via (at 108.0636 105.2) (size 0.6) (drill 0.3) (layers "F.Cu" "B.Cu") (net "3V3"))
 (segment (start 107.2 104.4) (end 107 104.4) (width 0.4) (layer "B.Cu") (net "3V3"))
 (segment (start 106.4322 102.0878) (end 106.52 102) (width 0.4) (layer "B.Cu") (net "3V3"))
 (segment (start 106.4322 103.8322) (end 106.4322 102.0878) (width 0.4) (layer "B.Cu") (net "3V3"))
 (segment (start 108.0636 105.2) (end 108.0636 104.9614) (width 0.4) (layer "B.Cu") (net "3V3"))
 (segment (start 107.2 105.2) (end 107.2 104.4) (width 0.4) (layer "B.Cu") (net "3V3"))
 (segment (start 107 104.4) (end 106.4322 103.8322) (width 0.4) (layer "B.Cu") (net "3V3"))
 (segment (start 107.2 105.2) (end 108.0636 105.2) (width 0.4) (layer "B.Cu") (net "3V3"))
 (segment (start 108.0636 104.9614) (end 109.25 103.775) (width 0.4) (layer "B.Cu") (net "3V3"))
 (segment (start 106.5 108.2497) (end 106.3676 108.1173) (width 0.2) (layer "F.Cu") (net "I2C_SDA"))
 (segment (start 106.5 109.6) (end 106.5 108.2497) (width 0.2) (layer "F.Cu") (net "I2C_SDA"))
 (via (at 106.3676 108.1173) (size 0.6) (drill 0.3) (layers "F.Cu" "B.Cu") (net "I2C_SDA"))
 (segment (start 104.8 106.8) (end 105.0503 106.8) (width 0.2) (layer "B.Cu") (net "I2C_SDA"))
 (segment (start 105.0503 106.8) (end 106.3676 108.1173) (width 0.2) (layer "B.Cu") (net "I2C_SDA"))
 (segment (start 107.9682 108.0103) (end 107.5 108.4785) (width 0.2) (layer "F.Cu") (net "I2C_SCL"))
 (segment (start 107.5 108.4785) (end 107.5 109.6) (width 0.2) (layer "F.Cu") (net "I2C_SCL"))
 (via (at 107.9682 108.0103) (size 0.6) (drill 0.3) (layers "F.Cu" "B.Cu") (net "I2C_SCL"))
 (segment (start 106.1475 108.8657) (end 107.6101 108.8657) (width 0.2) (layer "B.Cu") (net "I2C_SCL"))
 (segment (start 107.9682 108.5076) (end 107.9682 108.0103) (width 0.2) (layer "B.Cu") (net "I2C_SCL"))
 (segment (start 104.8818 107.6) (end 106.1475 108.8657) (width 0.2) (layer "B.Cu") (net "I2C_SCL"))
 (segment (start 104.8 107.6) (end 104.8818 107.6) (width 0.2) (layer "B.Cu") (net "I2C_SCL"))
 (segment (start 107.6101 108.8657) (end 107.9682 108.5076) (width 0.2) (layer "B.Cu") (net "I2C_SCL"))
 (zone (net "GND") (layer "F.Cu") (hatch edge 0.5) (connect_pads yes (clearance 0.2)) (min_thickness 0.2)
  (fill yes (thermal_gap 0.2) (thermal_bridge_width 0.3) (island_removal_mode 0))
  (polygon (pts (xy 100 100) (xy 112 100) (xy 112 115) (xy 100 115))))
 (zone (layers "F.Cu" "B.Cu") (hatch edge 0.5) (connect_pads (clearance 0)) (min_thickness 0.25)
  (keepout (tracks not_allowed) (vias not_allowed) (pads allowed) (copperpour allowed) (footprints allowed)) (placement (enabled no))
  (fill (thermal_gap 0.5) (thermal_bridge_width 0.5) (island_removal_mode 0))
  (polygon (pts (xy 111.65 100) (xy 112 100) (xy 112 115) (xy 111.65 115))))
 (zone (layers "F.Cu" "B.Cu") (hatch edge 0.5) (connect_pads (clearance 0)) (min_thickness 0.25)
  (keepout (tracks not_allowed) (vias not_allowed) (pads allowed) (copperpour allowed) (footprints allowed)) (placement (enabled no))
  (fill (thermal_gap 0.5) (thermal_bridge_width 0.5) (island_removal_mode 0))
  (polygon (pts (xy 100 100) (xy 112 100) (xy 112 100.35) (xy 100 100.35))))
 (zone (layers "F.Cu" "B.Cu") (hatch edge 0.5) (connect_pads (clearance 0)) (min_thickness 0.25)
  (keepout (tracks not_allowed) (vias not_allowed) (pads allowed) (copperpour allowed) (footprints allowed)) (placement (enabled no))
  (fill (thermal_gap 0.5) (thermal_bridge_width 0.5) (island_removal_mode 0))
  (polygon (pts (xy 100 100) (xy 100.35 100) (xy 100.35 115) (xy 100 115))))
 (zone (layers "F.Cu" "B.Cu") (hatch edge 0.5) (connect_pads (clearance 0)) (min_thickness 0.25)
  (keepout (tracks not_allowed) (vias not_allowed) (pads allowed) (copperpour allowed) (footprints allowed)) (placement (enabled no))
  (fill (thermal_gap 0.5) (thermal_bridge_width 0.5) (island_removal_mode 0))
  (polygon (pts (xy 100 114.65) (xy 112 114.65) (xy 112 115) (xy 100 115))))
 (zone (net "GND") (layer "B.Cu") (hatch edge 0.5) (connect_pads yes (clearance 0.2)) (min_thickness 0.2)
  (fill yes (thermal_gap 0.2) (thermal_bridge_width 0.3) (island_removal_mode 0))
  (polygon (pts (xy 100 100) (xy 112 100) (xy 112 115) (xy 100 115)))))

